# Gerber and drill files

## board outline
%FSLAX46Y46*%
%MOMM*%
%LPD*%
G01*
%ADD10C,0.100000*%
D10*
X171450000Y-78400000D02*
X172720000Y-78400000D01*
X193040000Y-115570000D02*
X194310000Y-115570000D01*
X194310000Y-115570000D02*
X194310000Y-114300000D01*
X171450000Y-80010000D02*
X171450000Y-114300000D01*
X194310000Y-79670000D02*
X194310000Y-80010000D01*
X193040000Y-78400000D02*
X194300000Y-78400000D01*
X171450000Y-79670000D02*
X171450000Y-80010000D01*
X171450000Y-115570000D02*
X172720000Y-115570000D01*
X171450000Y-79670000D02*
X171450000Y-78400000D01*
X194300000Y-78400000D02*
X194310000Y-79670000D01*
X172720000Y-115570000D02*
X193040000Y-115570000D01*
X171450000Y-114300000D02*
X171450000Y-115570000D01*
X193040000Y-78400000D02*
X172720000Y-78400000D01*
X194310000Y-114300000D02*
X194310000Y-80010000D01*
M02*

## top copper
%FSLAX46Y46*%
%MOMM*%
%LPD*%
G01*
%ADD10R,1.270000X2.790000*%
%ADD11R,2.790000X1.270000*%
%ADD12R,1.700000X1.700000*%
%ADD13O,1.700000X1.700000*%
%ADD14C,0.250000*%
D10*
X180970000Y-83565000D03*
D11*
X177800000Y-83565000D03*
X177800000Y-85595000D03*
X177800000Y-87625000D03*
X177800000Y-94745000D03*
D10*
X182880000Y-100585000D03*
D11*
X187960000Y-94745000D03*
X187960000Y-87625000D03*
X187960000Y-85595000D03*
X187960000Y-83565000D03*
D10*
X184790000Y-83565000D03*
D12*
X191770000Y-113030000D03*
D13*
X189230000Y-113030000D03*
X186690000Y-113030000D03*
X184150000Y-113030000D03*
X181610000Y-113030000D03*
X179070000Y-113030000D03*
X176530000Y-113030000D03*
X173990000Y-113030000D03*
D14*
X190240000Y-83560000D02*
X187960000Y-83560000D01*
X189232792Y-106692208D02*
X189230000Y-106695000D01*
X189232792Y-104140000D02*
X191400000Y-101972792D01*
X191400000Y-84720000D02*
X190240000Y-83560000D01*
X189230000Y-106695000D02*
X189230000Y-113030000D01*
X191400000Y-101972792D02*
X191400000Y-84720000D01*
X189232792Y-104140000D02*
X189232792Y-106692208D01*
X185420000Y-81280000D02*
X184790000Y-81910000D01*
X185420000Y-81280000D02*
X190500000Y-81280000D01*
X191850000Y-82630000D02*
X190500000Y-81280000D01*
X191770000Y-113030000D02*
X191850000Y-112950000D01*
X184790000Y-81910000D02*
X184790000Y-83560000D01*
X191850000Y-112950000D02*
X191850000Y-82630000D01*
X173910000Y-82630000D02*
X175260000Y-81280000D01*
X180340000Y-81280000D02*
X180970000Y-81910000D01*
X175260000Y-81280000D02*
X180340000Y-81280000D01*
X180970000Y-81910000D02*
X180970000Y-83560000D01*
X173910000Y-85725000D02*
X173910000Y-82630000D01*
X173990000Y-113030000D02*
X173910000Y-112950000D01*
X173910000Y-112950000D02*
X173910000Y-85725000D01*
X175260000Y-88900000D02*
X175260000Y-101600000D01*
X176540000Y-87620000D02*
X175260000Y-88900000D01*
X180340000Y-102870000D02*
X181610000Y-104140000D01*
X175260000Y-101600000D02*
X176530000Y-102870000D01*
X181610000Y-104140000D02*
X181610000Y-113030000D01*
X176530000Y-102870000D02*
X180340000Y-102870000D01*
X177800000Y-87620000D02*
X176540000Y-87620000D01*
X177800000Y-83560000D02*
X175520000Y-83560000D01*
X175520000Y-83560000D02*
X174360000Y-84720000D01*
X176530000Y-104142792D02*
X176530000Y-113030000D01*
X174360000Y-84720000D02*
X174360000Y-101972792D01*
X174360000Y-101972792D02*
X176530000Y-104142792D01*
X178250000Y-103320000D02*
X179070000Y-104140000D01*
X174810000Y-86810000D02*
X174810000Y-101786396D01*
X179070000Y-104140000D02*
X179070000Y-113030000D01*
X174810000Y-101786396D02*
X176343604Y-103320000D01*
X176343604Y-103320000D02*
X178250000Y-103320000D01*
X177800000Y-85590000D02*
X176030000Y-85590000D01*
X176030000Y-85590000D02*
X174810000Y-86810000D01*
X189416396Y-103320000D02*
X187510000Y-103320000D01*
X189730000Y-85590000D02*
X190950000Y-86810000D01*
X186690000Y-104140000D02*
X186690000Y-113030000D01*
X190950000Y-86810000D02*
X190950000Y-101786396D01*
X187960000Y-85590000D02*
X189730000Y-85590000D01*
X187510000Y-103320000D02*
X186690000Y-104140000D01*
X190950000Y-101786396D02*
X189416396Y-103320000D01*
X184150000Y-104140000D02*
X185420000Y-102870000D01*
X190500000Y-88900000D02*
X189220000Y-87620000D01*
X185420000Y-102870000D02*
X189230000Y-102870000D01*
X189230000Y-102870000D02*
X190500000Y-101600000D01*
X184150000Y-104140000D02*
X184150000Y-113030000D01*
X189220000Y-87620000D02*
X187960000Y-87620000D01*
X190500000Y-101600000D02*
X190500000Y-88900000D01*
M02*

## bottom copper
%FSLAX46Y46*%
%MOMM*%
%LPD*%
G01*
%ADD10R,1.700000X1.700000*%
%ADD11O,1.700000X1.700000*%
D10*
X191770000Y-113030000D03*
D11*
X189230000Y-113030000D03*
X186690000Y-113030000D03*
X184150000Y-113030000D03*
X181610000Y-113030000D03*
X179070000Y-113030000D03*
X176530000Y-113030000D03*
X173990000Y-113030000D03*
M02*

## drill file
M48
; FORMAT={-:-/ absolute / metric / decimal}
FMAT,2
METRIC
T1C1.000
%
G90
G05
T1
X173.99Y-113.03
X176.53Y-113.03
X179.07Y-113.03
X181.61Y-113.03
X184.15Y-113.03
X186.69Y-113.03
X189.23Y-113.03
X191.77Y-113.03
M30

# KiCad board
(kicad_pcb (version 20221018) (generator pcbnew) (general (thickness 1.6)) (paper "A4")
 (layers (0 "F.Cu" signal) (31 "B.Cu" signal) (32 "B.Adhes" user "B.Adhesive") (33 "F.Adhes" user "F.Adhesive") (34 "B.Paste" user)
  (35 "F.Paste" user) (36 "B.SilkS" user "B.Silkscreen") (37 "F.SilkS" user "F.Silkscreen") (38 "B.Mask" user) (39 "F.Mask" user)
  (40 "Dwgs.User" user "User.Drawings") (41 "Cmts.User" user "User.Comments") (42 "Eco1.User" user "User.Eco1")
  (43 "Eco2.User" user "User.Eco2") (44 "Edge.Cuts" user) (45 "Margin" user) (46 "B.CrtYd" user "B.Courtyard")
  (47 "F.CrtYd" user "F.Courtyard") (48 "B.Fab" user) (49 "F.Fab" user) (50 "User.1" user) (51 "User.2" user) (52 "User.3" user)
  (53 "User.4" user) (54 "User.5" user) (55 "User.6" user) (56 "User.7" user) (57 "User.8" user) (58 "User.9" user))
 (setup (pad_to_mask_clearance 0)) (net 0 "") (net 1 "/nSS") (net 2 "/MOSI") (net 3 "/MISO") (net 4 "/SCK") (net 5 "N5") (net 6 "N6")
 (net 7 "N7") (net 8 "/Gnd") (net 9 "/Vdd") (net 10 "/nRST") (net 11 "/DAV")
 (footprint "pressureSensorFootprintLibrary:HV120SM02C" (layer "F.Cu") (at 182.88 92.075 90)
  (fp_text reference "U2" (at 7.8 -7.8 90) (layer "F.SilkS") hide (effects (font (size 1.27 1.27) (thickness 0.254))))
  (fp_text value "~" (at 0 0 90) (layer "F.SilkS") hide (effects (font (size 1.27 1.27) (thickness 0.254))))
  (pad "1" smd rect (at 8.51 -1.91 180) (size 1.27 2.79) (layers "F.Cu" "F.Paste" "F.Mask") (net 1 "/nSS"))
  (pad "2" smd rect (at 8.51 -5.08 90) (size 1.27 2.79) (layers "F.Cu" "F.Paste" "F.Mask") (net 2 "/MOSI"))
  (pad "3" smd rect (at 6.48 -5.08 90) (size 1.27 2.79) (layers "F.Cu" "F.Paste" "F.Mask") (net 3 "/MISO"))
  (pad "4" smd rect (at 4.45 -5.08 90) (size 1.27 2.79) (layers "F.Cu" "F.Paste" "F.Mask") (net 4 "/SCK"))
  (pad "5" smd rect (at -2.67 -5.08 90) (size 1.27 2.79) (layers "F.Cu" "F.Paste" "F.Mask") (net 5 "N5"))
  (pad "6" smd rect (at -8.51 0 180) (size 1.27 2.79) (layers "F.Cu" "F.Paste" "F.Mask") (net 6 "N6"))
  (pad "7" smd rect (at -2.67 5.08 90) (size 1.27 2.79) (layers "F.Cu" "F.Paste" "F.Mask") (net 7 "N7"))
  (pad "8" smd rect (at 4.45 5.08 90) (size 1.27 2.79) (layers "F.Cu" "F.Paste" "F.Mask") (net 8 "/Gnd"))
  (pad "9" smd rect (at 6.48 5.08 90) (size 1.27 2.79) (layers "F.Cu" "F.Paste" "F.Mask") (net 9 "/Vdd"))
  (pad "10" smd rect (at 8.51 5.08 90) (size 1.27 2.79) (layers "F.Cu" "F.Paste" "F.Mask") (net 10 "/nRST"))
  (pad "11" smd rect (at 8.51 1.91 180) (size 1.27 2.79) (layers "F.Cu" "F.Paste" "F.Mask") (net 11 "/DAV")))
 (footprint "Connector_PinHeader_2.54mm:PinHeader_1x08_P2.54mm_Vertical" (layer "B.Cu") (at 191.77 113.03 90)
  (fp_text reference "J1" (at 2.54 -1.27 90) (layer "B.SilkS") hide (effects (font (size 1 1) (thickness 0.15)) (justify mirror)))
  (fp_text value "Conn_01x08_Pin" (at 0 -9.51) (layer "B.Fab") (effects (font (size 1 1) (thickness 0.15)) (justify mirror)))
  (pad "1" thru_hole rect (at 0 0 90) (size 1.7 1.7) (drill 1) (layers "*.Cu" "*.Mask") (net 11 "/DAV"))
  (pad "2" thru_hole oval (at 0 -2.54 90) (size 1.7 1.7) (drill 1) (layers "*.Cu" "*.Mask") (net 10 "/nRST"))
  (pad "3" thru_hole oval (at 0 -5.08 90) (size 1.7 1.7) (drill 1) (layers "*.Cu" "*.Mask") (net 9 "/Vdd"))
  (pad "4" thru_hole oval (at 0 -7.62 90) (size 1.7 1.7) (drill 1) (layers "*.Cu" "*.Mask") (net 8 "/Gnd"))
  (pad "5" thru_hole oval (at 0 -10.16 90) (size 1.7 1.7) (drill 1) (layers "*.Cu" "*.Mask") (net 4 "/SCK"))
  (pad "6" thru_hole oval (at 0 -12.7 90) (size 1.7 1.7) (drill 1) (layers "*.Cu" "*.Mask") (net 3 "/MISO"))
  (pad "7" thru_hole oval (at 0 -15.24 90) (size 1.7 1.7) (drill 1) (layers "*.Cu" "*.Mask") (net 2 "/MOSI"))
  (pad "8" thru_hole oval (at 0 -17.78 90) (size 1.7 1.7) (drill 1) (layers "*.Cu" "*.Mask") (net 1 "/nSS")))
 (gr_line (start 171.45 78.4) (end 172.72 78.4) (stroke (width 0.1) (type default)) (layer "Edge.Cuts"))
 (gr_line (start 193.04 115.57) (end 194.31 115.57) (stroke (width 0.1) (type default)) (layer "Edge.Cuts"))
 (gr_line (start 194.31 115.57) (end 194.31 114.3) (stroke (width 0.1) (type default)) (layer "Edge.Cuts"))
 (gr_line (start 171.45 80.01) (end 171.45 114.3) (stroke (width 0.1) (type default)) (layer "Edge.Cuts"))
 (gr_line (start 194.31 79.67) (end 194.31 80.01) (stroke (width 0.1) (type default)) (layer "Edge.Cuts"))
 (gr_line (start 193.04 78.4) (end 194.3 78.4) (stroke (width 0.1) (type default)) (layer "Edge.Cuts"))
 (gr_line (start 171.45 79.67) (end 171.45 80.01) (stroke (width 0.1) (type default)) (layer "Edge.Cuts"))
 (gr_line (start 171.45 115.57) (end 172.72 115.57) (stroke (width 0.1) (type default)) (layer "Edge.Cuts"))
 (gr_line (start 171.45 79.67) (end 171.45 78.4) (stroke (width 0.1) (type default)) (layer "Edge.Cuts"))
 (gr_line (start 194.3 78.4) (end 194.31 79.67) (stroke (width 0.1) (type default)) (layer "Edge.Cuts"))
 (gr_line (start 172.72 115.57) (end 193.04 115.57) (stroke (width 0.1) (type default)) (layer "Edge.Cuts"))
 (gr_line (start 171.45 114.3) (end 171.45 115.57) (stroke (width 0.1) (type default)) (layer "Edge.Cuts"))
 (gr_line (start 193.04 78.4) (end 172.72 78.4) (stroke (width 0.1) (type default)) (layer "Edge.Cuts"))
 (gr_line (start 194.31 114.3) (end 194.31 80.01) (stroke (width 0.1) (type default)) (layer "Edge.Cuts"))
 (segment (start 190.24 83.56) (end 187.96 83.56) (width 0.25) (layer "F.Cu") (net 10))
 (segment (start 189.232792 106.692208) (end 189.23 106.695) (width 0.25) (layer "F.Cu") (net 10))
 (segment (start 189.232792 104.14) (end 191.4 101.972792) (width 0.25) (layer "F.Cu") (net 10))
 (segment (start 191.4 84.72) (end 190.24 83.56) (width 0.25) (layer "F.Cu") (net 10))
 (segment (start 189.23 106.695) (end 189.23 113.03) (width 0.25) (layer "F.Cu") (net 10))
 (segment (start 191.4 101.972792) (end 191.4 84.72) (width 0.25) (layer "F.Cu") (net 10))
 (segment (start 189.232792 104.14) (end 189.232792 106.692208) (width 0.25) (layer "F.Cu") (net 10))
 (segment (start 185.42 81.28) (end 184.79 81.91) (width 0.25) (layer "F.Cu") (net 11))
 (segment (start 185.42 81.28) (end 190.5 81.28) (width 0.25) (layer "F.Cu") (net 11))
 (segment (start 191.85 82.63) (end 190.5 81.28) (width 0.25) (layer "F.Cu") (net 11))
 (segment (start 191.77 113.03) (end 191.85 112.95) (width 0.25) (layer "F.Cu") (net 11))
 (segment (start 184.79 81.91) (end 184.79 83.56) (width 0.25) (layer "F.Cu") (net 11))
 (segment (start 191.85 112.95) (end 191.85 82.63) (width 0.25) (layer "F.Cu") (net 11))
 (segment (start 173.91 82.63) (end 175.26 81.28) (width 0.25) (layer "F.Cu") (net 1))
 (segment (start 180.34 81.28) (end 180.97 81.91) (width 0.25) (layer "F.Cu") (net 1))
 (segment (start 175.26 81.28) (end 180.34 81.28) (width 0.25) (layer "F.Cu") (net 1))
 (segment (start 180.97 81.91) (end 180.97 83.56) (width 0.25) (layer "F.Cu") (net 1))
 (segment (start 173.91 85.725) (end 173.91 82.63) (width 0.25) (layer "F.Cu") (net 1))
 (segment (start 173.99 113.03) (end 173.91 112.95) (width 0.25) (layer "F.Cu") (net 1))
 (segment (start 173.91 112.95) (end 173.91 85.725) (width 0.25) (layer "F.Cu") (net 1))
 (segment (start 175.26 88.9) (end 175.26 101.6) (width 0.25) (layer "F.Cu") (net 4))
 (segment (start 176.54 87.62) (end 175.26 88.9) (width 0.25) (layer "F.Cu") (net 4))
 (segment (start 180.34 102.87) (end 181.61 104.14) (width 0.25) (layer "F.Cu") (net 4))
 (segment (start 175.26 101.6) (end 176.53 102.87) (width 0.25) (layer "F.Cu") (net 4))
 (segment (start 181.61 104.14) (end 181.61 113.03) (width 0.25) (layer "F.Cu") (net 4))
 (segment (start 176.53 102.87) (end 180.34 102.87) (width 0.25) (layer "F.Cu") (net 4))
 (segment (start 177.8 87.62) (end 176.54 87.62) (width 0.25) (layer "F.Cu") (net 4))
 (segment (start 177.8 83.56) (end 175.52 83.56) (width 0.25) (layer "F.Cu") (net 2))
 (segment (start 175.52 83.56) (end 174.36 84.72) (width 0.25) (layer "F.Cu") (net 2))
 (segment (start 176.53 104.142792) (end 176.53 113.03) (width 0.25) (layer "F.Cu") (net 2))
 (segment (start 174.36 84.72) (end 174.36 101.972792) (width 0.25) (layer "F.Cu") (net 2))
 (segment (start 174.36 101.972792) (end 176.53 104.142792) (width 0.25) (layer "F.Cu") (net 2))
 (segment (start 178.25 103.32) (end 179.07 104.14) (width 0.25) (layer "F.Cu") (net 3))
 (segment (start 174.81 86.81) (end 174.81 101.786396) (width 0.25) (layer "F.Cu") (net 3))
 (segment (start 179.07 104.14) (end 179.07 113.03) (width 0.25) (layer "F.Cu") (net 3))
 (segment (start 174.81 101.786396) (end 176.343604 103.32) (width 0.25) (layer "F.Cu") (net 3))
 (segment (start 176.343604 103.32) (end 178.25 103.32) (width 0.25) (layer "F.Cu") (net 3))
 (segment (start 177.8 85.59) (end 176.03 85.59) (width 0.25) (layer "F.Cu") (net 3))
 (segment (start 176.03 85.59) (end 174.81 86.81) (width 0.25) (layer "F.Cu") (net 3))
 (segment (start 189.416396 103.32) (end 187.51 103.32) (width 0.25) (layer "F.Cu") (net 9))
 (segment (start 189.73 85.59) (end 190.95 86.81) (width 0.25) (layer "F.Cu") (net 9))
 (segment (start 186.69 104.14) (end 186.69 113.03) (width 0.25) (layer "F.Cu") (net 9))
 (segment (start 190.95 86.81) (end 190.95 101.786396) (width 0.25) (layer "F.Cu") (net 9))
 (segment (start 187.96 85.59) (end 189.73 85.59) (width 0.25) (layer "F.Cu") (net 9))
 (segment (start 187.51 103.32) (end 186.69 104.14) (width 0.25) (layer "F.Cu") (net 9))
 (segment (start 190.95 101.786396) (end 189.416396 103.32) (width 0.25) (layer "F.Cu") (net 9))
 (segment (start 184.15 104.14) (end 185.42 102.87) (width 0.25) (layer "F.Cu") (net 8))
 (segment (start 190.5 88.9) (end 189.22 87.62) (width 0.25) (layer "F.Cu") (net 8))
 (segment (start 185.42 102.87) (end 189.23 102.87) (width 0.25) (layer "F.Cu") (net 8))
 (segment (start 189.23 102.87) (end 190.5 101.6) (width 0.25) (layer "F.Cu") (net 8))
 (segment (start 184.15 104.14) (end 184.15 113.03) (width 0.25) (layer "F.Cu") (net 8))
 (segment (start 189.22 87.62) (end 187.96 87.62) (width 0.25) (layer "F.Cu") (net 8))
 (segment (start 190.5 101.6) (end 190.5 88.9) (width 0.25) (layer "F.Cu") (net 8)))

